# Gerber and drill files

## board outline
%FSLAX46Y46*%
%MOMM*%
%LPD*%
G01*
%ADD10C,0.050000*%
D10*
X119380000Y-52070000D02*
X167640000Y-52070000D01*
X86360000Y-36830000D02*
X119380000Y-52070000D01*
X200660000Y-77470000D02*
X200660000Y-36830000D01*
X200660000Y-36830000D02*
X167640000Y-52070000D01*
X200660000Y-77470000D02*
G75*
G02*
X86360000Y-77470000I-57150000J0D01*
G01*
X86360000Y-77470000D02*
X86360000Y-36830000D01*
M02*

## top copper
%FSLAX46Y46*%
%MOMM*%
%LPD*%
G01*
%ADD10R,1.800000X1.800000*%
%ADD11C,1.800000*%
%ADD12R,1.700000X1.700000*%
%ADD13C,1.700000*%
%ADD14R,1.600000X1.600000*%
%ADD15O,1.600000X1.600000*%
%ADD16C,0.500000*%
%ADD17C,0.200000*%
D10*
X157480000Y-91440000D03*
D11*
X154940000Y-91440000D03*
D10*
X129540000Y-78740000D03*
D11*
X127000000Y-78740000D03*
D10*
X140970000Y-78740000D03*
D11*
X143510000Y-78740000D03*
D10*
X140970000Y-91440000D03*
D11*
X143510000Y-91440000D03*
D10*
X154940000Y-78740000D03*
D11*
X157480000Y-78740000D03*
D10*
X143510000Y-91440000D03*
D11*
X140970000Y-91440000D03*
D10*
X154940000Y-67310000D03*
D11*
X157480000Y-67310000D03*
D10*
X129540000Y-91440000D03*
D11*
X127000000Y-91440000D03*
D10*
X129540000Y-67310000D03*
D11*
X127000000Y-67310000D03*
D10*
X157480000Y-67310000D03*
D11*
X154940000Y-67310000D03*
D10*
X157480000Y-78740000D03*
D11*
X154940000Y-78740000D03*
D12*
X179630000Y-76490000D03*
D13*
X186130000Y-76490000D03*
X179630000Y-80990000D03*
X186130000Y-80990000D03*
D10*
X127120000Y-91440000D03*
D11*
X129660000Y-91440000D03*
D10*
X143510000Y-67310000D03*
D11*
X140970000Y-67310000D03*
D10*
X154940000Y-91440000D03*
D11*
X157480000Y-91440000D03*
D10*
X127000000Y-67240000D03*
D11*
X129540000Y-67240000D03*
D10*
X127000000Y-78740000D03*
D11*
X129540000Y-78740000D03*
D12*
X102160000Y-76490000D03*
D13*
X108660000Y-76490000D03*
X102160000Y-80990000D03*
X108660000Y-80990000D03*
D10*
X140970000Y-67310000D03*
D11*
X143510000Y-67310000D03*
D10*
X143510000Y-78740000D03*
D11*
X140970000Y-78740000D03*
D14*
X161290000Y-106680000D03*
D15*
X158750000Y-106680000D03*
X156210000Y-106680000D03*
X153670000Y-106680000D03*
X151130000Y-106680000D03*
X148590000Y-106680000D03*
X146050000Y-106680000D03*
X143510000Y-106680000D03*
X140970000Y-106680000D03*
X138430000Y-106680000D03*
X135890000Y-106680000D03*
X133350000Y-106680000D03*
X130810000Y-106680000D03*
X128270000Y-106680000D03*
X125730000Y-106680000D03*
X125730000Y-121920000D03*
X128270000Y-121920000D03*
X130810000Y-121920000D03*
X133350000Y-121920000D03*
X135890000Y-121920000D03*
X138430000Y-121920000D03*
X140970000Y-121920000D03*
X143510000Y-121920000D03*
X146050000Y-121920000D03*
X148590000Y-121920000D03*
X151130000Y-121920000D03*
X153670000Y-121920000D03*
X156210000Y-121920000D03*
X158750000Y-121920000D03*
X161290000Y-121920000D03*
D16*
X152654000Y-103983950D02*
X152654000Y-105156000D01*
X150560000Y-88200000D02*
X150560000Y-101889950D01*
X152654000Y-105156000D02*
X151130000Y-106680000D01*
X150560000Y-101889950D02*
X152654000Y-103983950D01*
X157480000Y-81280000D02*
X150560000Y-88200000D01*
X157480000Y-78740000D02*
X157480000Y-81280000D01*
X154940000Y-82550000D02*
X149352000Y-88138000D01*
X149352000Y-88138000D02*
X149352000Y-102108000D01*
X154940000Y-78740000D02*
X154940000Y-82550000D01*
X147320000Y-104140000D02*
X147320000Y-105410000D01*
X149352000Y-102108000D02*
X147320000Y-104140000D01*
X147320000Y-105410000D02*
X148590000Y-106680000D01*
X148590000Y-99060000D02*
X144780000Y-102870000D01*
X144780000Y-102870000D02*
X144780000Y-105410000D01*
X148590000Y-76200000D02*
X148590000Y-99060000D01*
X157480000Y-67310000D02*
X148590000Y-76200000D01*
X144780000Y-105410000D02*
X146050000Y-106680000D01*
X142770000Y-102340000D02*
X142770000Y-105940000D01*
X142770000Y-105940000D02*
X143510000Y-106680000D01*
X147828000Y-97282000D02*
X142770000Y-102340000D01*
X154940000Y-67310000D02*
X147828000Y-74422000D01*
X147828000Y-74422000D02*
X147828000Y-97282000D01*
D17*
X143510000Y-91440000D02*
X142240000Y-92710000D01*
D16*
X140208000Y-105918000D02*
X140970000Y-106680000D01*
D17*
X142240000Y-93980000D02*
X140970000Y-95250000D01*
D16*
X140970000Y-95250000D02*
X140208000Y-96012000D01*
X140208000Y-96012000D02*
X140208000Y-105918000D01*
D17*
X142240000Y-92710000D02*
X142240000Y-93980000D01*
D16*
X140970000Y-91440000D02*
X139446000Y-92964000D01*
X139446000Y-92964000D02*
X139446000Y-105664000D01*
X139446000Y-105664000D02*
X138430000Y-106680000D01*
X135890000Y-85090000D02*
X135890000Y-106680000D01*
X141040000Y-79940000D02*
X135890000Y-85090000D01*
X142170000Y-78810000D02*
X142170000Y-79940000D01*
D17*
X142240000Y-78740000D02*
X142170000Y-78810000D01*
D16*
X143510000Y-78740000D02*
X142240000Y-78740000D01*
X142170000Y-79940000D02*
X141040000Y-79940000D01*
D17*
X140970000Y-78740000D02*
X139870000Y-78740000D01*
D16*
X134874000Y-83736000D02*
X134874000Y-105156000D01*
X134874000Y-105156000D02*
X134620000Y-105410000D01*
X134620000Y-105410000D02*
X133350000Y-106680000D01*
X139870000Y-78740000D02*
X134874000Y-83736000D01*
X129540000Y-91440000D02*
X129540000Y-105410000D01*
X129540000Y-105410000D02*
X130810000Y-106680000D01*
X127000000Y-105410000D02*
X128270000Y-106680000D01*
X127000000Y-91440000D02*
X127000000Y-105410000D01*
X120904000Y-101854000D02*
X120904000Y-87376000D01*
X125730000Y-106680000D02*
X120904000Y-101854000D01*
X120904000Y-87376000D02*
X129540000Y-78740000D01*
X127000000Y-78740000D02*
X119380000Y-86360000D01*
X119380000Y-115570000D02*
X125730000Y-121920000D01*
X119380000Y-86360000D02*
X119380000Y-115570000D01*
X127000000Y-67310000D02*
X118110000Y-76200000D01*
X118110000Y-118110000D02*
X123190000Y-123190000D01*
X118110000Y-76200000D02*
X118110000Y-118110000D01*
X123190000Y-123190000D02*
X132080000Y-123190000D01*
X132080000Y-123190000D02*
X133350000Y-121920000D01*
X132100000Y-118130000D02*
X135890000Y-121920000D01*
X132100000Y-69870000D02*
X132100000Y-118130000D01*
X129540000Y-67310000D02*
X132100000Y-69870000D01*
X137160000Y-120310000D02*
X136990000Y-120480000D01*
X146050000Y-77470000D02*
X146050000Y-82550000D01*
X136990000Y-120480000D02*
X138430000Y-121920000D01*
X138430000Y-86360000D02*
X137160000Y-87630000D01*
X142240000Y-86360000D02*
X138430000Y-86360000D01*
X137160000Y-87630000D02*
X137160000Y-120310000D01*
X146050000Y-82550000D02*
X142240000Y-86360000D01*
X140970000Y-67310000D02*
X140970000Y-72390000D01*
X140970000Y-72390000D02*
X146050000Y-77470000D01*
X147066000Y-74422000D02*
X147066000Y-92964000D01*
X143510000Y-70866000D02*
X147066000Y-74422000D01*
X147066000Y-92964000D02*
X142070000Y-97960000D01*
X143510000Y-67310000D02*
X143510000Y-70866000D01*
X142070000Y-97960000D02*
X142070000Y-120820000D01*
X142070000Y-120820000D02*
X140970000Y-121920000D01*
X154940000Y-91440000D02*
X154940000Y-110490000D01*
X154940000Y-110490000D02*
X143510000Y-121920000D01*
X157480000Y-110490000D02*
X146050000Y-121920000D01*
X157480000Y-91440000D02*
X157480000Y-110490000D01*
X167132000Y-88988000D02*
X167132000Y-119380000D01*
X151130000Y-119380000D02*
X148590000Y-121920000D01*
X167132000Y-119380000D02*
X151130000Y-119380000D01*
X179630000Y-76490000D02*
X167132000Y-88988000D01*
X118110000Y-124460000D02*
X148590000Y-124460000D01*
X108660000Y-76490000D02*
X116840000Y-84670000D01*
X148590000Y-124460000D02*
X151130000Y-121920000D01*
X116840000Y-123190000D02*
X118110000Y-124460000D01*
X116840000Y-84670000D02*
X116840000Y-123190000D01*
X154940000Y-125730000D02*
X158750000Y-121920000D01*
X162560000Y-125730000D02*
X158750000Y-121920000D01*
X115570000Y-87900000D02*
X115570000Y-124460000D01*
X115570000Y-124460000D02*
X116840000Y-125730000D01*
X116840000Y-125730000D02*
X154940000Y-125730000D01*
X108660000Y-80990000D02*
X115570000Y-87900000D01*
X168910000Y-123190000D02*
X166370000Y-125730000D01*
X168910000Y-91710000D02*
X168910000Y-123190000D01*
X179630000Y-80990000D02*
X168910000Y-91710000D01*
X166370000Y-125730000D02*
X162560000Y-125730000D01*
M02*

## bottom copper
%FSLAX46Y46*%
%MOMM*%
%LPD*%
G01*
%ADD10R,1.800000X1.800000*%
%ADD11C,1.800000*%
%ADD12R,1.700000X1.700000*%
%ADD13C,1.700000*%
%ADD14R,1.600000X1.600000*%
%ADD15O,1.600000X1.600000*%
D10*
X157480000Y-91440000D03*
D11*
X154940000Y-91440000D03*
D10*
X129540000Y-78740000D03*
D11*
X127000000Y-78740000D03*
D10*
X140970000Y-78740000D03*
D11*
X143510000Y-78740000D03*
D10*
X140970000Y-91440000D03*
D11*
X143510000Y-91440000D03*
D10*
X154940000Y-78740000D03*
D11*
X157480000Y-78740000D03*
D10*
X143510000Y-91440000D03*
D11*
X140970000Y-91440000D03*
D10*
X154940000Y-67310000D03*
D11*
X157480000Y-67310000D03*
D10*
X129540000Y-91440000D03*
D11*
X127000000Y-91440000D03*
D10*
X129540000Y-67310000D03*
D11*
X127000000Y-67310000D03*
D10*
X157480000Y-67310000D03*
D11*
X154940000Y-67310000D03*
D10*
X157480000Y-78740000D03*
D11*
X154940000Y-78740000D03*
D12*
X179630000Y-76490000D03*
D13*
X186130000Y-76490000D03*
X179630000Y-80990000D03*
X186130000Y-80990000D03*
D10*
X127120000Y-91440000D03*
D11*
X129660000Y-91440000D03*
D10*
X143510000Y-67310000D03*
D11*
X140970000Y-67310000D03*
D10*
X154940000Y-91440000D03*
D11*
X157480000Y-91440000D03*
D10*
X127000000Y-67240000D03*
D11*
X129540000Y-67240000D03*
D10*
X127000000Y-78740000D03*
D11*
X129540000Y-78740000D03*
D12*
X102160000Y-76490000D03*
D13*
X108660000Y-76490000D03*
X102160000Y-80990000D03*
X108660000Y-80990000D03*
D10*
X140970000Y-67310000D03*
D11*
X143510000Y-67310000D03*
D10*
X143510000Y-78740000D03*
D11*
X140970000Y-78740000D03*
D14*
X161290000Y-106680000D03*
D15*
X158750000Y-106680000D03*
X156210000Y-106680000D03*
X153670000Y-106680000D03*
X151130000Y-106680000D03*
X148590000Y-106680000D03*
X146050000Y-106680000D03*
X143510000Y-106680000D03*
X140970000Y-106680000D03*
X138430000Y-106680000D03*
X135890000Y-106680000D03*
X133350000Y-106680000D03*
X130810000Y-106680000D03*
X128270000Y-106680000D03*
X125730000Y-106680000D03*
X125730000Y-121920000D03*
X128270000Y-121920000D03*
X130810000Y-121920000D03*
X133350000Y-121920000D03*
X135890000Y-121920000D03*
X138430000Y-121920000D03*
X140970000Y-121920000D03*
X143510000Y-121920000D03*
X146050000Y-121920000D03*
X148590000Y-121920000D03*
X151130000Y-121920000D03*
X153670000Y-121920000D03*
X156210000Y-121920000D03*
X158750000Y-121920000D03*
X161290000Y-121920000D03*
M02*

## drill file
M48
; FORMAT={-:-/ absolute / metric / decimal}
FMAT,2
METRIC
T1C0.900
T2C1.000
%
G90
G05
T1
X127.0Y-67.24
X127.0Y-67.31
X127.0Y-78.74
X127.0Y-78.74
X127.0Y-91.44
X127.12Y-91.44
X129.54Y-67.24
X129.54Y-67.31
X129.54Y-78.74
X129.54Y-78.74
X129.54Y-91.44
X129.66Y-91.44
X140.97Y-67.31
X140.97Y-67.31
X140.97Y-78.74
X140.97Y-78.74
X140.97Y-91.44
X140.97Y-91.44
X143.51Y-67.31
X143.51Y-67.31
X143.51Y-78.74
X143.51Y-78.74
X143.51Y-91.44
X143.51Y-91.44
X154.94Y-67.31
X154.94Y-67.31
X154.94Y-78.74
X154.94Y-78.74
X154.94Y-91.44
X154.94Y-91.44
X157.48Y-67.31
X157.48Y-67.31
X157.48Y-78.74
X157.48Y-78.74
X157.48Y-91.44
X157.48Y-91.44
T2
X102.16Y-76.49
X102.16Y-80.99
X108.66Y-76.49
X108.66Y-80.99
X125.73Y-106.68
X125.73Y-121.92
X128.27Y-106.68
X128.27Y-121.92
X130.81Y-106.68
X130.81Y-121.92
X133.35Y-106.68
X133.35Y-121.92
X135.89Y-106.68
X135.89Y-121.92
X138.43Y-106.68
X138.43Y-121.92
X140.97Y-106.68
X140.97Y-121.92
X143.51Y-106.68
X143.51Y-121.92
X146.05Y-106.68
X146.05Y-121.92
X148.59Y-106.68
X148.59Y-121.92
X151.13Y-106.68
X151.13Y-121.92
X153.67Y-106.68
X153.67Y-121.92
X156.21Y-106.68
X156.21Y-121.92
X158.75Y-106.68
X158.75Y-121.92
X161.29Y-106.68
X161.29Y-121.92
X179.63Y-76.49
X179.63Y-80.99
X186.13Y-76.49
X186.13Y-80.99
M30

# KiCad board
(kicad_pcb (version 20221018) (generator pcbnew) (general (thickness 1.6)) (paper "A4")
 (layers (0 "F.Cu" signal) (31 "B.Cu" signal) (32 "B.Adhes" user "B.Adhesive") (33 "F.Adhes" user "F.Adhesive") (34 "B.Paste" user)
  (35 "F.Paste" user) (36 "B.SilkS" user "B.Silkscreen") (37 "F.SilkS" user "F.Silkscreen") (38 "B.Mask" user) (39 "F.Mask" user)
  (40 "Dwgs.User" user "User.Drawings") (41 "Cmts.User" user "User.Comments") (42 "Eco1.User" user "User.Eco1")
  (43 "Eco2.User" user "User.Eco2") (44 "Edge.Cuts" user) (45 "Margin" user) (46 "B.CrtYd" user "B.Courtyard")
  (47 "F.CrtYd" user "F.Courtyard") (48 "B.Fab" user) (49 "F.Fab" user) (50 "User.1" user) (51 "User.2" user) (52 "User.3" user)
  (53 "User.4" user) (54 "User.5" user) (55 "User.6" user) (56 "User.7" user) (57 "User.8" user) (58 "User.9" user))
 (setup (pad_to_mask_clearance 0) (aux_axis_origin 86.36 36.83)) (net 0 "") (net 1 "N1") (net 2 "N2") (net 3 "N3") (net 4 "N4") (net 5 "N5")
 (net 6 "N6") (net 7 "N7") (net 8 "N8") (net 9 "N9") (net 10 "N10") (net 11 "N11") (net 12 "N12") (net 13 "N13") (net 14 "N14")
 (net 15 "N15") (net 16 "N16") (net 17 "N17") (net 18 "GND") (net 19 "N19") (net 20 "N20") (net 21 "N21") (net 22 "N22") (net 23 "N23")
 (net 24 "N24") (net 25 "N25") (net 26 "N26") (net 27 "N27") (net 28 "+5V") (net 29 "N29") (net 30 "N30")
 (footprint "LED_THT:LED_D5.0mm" (layer "F.Cu") (at 157.48 91.44 180)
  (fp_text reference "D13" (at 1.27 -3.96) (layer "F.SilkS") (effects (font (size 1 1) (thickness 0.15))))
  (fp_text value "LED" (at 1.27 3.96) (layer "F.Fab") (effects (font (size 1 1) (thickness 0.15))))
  (pad "1" thru_hole rect (at 0 0 180) (size 1.8 1.8) (drill 0.9) (layers "*.Cu" "*.Mask") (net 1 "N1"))
  (pad "2" thru_hole circle (at 2.54 0 180) (size 1.8 1.8) (drill 0.9) (layers "*.Cu" "*.Mask") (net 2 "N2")))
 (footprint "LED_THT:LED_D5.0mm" (layer "F.Cu") (at 129.54 78.74 180)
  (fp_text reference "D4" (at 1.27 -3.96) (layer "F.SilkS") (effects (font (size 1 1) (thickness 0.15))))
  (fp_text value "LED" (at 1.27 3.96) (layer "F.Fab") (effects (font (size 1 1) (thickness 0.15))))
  (pad "1" thru_hole rect (at 0 0 180) (size 1.8 1.8) (drill 0.9) (layers "*.Cu" "*.Mask") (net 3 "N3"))
  (pad "2" thru_hole circle (at 2.54 0 180) (size 1.8 1.8) (drill 0.9) (layers "*.Cu" "*.Mask") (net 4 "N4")))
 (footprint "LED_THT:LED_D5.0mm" (layer "F.Cu") (at 140.97 78.74)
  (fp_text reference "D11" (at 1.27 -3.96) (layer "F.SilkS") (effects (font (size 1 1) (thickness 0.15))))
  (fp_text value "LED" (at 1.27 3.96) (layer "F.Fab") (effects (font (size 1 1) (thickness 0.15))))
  (pad "1" thru_hole rect (at 0 0) (size 1.8 1.8) (drill 0.9) (layers "*.Cu" "*.Mask") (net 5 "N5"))
  (pad "2" thru_hole circle (at 2.54 0) (size 1.8 1.8) (drill 0.9) (layers "*.Cu" "*.Mask") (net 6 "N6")))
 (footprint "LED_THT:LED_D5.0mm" (layer "F.Cu") (at 140.97 91.44)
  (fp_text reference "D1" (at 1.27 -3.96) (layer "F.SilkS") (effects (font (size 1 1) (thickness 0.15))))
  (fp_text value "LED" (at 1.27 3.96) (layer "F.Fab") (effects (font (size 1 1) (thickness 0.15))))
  (pad "1" thru_hole rect (at 0 0) (size 1.8 1.8) (drill 0.9) (layers "*.Cu" "*.Mask") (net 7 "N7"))
  (pad "2" thru_hole circle (at 2.54 0) (size 1.8 1.8) (drill 0.9) (layers "*.Cu" "*.Mask") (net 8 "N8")))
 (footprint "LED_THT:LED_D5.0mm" (layer "F.Cu") (at 154.94 78.74)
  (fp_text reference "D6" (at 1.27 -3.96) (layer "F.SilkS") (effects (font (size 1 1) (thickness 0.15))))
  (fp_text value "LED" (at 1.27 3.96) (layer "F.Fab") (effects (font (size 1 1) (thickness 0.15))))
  (pad "1" thru_hole rect (at 0 0) (size 1.8 1.8) (drill 0.9) (layers "*.Cu" "*.Mask") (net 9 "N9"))
  (pad "2" thru_hole circle (at 2.54 0) (size 1.8 1.8) (drill 0.9) (layers "*.Cu" "*.Mask") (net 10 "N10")))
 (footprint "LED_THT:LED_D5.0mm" (layer "F.Cu") (at 143.51 91.44 180)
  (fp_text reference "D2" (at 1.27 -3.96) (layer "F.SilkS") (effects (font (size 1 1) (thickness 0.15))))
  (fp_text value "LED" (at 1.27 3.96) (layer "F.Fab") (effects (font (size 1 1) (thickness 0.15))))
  (pad "1" thru_hole rect (at 0 0 180) (size 1.8 1.8) (drill 0.9) (layers "*.Cu" "*.Mask") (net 8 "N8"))
  (pad "2" thru_hole circle (at 2.54 0 180) (size 1.8 1.8) (drill 0.9) (layers "*.Cu" "*.Mask") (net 7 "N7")))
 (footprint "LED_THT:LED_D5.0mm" (layer "F.Cu") (at 154.94 67.31)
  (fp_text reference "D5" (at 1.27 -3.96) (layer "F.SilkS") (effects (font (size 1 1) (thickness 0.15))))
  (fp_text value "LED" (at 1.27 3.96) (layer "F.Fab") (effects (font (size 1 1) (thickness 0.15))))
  (pad "1" thru_hole rect (at 0 0) (size 1.8 1.8) (drill 0.9) (layers "*.Cu" "*.Mask") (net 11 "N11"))
  (pad "2" thru_hole circle (at 2.54 0) (size 1.8 1.8) (drill 0.9) (layers "*.Cu" "*.Mask") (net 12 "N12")))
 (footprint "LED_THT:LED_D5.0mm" (layer "F.Cu") (at 129.54 91.44 180)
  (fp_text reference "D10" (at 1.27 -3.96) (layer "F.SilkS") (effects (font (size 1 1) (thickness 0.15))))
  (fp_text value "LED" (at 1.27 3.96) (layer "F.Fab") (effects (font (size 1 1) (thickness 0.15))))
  (pad "1" thru_hole rect (at 0 0 180) (size 1.8 1.8) (drill 0.9) (layers "*.Cu" "*.Mask") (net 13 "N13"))
  (pad "2" thru_hole circle (at 2.54 0 180) (size 1.8 1.8) (drill 0.9) (layers "*.Cu" "*.Mask") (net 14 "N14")))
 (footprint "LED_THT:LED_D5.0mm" (layer "F.Cu") (at 129.54 67.31 180)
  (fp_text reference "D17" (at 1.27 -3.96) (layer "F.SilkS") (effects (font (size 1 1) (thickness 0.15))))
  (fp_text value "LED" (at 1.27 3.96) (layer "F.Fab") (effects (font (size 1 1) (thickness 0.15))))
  (pad "1" thru_hole rect (at 0 0 180) (size 1.8 1.8) (drill 0.9) (layers "*.Cu" "*.Mask") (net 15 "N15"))
  (pad "2" thru_hole circle (at 2.54 0 180) (size 1.8 1.8) (drill 0.9) (layers "*.Cu" "*.Mask") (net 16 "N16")))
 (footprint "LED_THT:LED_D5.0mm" (layer "F.Cu") (at 157.48 67.31 180)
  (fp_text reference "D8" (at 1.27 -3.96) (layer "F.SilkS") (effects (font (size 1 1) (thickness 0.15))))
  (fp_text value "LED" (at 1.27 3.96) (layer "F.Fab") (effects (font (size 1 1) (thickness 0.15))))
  (pad "1" thru_hole rect (at 0 0 180) (size 1.8 1.8) (drill 0.9) (layers "*.Cu" "*.Mask") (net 12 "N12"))
  (pad "2" thru_hole circle (at 2.54 0 180) (size 1.8 1.8) (drill 0.9) (layers "*.Cu" "*.Mask") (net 11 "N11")))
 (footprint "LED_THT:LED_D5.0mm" (layer "F.Cu") (at 157.48 78.74 180)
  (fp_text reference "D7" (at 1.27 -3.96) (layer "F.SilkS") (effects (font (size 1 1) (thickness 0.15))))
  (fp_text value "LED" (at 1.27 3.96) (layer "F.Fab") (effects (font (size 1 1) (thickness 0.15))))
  (pad "1" thru_hole rect (at 0 0 180) (size 1.8 1.8) (drill 0.9) (layers "*.Cu" "*.Mask") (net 10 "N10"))
  (pad "2" thru_hole circle (at 2.54 0 180) (size 1.8 1.8) (drill 0.9) (layers "*.Cu" "*.Mask") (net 9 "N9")))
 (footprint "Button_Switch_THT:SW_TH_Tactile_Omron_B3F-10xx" (layer "F.Cu") (at 179.63 76.49)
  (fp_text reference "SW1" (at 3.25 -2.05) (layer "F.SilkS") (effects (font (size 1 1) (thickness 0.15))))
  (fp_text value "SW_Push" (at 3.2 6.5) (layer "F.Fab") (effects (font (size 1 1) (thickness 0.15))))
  (pad "1" thru_hole rect (at 0 0) (size 1.7 1.7) (drill 1) (layers "*.Cu" "*.Mask") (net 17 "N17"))
  (pad "1" thru_hole circle (at 6.5 0) (size 1.7 1.7) (drill 1) (layers "*.Cu" "*.Mask") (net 17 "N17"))
  (pad "2" thru_hole circle (at 0 4.5) (size 1.7 1.7) (drill 1) (layers "*.Cu" "*.Mask") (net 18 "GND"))
  (pad "2" thru_hole circle (at 6.5 4.5) (size 1.7 1.7) (drill 1) (layers "*.Cu" "*.Mask") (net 18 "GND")))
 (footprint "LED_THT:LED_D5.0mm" (layer "F.Cu") (at 127.12 91.44)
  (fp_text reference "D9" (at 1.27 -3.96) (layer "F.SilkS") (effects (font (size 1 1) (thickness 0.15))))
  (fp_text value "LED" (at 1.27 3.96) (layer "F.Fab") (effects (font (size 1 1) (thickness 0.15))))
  (pad "1" thru_hole rect (at 0 0) (size 1.8 1.8) (drill 0.9) (layers "*.Cu" "*.Mask") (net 14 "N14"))
  (pad "2" thru_hole circle (at 2.54 0) (size 1.8 1.8) (drill 0.9) (layers "*.Cu" "*.Mask") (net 13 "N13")))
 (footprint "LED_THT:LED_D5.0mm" (layer "F.Cu") (at 143.51 67.31 180)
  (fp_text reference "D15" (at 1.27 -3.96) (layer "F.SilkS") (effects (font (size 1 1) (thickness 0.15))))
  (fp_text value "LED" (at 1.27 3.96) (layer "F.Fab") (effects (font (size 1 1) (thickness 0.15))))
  (pad "1" thru_hole rect (at 0 0 180) (size 1.8 1.8) (drill 0.9) (layers "*.Cu" "*.Mask") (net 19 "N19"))
  (pad "2" thru_hole circle (at 2.54 0 180) (size 1.8 1.8) (drill 0.9) (layers "*.Cu" "*.Mask") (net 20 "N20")))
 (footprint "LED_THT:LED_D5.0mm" (layer "F.Cu") (at 154.94 91.44)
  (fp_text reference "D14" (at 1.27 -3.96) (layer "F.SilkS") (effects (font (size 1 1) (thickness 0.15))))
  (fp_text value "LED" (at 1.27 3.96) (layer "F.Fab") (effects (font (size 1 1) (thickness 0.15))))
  (pad "1" thru_hole rect (at 0 0) (size 1.8 1.8) (drill 0.9) (layers "*.Cu" "*.Mask") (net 2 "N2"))
  (pad "2" thru_hole circle (at 2.54 0) (size 1.8 1.8) (drill 0.9) (layers "*.Cu" "*.Mask") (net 1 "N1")))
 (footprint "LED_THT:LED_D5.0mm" (layer "F.Cu") (at 127 67.24)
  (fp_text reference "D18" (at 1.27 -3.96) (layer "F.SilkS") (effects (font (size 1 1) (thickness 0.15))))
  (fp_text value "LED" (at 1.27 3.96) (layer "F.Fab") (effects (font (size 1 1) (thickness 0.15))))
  (pad "1" thru_hole rect (at 0 0) (size 1.8 1.8) (drill 0.9) (layers "*.Cu" "*.Mask") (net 16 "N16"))
  (pad "2" thru_hole circle (at 2.54 0) (size 1.8 1.8) (drill 0.9) (layers "*.Cu" "*.Mask") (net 15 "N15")))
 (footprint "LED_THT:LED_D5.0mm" (layer "F.Cu") (at 127 78.74)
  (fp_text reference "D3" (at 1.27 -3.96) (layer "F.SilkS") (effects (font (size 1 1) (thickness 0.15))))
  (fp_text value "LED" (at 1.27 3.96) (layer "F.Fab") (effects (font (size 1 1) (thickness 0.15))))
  (pad "1" thru_hole rect (at 0 0) (size 1.8 1.8) (drill 0.9) (layers "*.Cu" "*.Mask") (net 4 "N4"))
  (pad "2" thru_hole circle (at 2.54 0) (size 1.8 1.8) (drill 0.9) (layers "*.Cu" "*.Mask") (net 3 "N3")))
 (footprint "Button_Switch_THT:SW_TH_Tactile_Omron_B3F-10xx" (layer "F.Cu") (at 102.16 76.49)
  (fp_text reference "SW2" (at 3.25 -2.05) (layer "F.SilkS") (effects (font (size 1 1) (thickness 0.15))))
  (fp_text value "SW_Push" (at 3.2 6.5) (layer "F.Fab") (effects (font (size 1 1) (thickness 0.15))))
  (pad "1" thru_hole rect (at 0 0) (size 1.7 1.7) (drill 1) (layers "*.Cu" "*.Mask") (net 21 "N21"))
  (pad "1" thru_hole circle (at 6.5 0) (size 1.7 1.7) (drill 1) (layers "*.Cu" "*.Mask") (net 21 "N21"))
  (pad "2" thru_hole circle (at 0 4.5) (size 1.7 1.7) (drill 1) (layers "*.Cu" "*.Mask") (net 18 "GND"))
  (pad "2" thru_hole circle (at 6.5 4.5) (size 1.7 1.7) (drill 1) (layers "*.Cu" "*.Mask") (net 18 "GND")))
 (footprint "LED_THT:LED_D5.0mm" (layer "F.Cu") (at 140.97 67.31)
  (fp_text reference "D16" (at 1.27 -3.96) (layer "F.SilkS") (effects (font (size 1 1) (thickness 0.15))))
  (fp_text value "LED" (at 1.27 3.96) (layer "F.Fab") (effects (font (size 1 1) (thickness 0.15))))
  (pad "1" thru_hole rect (at 0 0) (size 1.8 1.8) (drill 0.9) (layers "*.Cu" "*.Mask") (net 20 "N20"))
  (pad "2" thru_hole circle (at 2.54 0) (size 1.8 1.8) (drill 0.9) (layers "*.Cu" "*.Mask") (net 19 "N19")))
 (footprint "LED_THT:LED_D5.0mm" (layer "F.Cu") (at 143.51 78.74 180)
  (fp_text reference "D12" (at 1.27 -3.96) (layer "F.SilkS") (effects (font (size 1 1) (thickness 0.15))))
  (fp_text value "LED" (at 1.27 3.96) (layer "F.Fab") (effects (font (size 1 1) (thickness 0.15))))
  (pad "1" thru_hole rect (at 0 0 180) (size 1.8 1.8) (drill 0.9) (layers "*.Cu" "*.Mask") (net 6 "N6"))
  (pad "2" thru_hole circle (at 2.54 0 180) (size 1.8 1.8) (drill 0.9) (layers "*.Cu" "*.Mask") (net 5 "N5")))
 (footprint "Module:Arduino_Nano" (layer "F.Cu") (at 161.29 106.68 -90)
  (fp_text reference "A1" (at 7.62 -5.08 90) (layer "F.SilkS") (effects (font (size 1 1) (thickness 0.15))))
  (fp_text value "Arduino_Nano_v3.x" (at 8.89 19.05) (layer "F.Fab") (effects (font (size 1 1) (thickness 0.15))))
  (pad "1" thru_hole rect (at 0 0 270) (size 1.6 1.6) (drill 1) (layers "*.Cu" "*.Mask") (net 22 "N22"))
  (pad "2" thru_hole oval (at 0 2.54 270) (size 1.6 1.6) (drill 1) (layers "*.Cu" "*.Mask") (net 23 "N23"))
  (pad "3" thru_hole oval (at 0 5.08 270) (size 1.6 1.6) (drill 1) (layers "*.Cu" "*.Mask") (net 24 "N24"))
  (pad "4" thru_hole oval (at 0 7.62 270) (size 1.6 1.6) (drill 1) (layers "*.Cu" "*.Mask") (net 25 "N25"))
  (pad "5" thru_hole oval (at 0 10.16 270) (size 1.6 1.6) (drill 1) (layers "*.Cu" "*.Mask") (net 10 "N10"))
  (pad "6" thru_hole oval (at 0 12.7 270) (size 1.6 1.6) (drill 1) (layers "*.Cu" "*.Mask") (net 9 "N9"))
  (pad "7" thru_hole oval (at 0 15.24 270) (size 1.6 1.6) (drill 1) (layers "*.Cu" "*.Mask") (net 12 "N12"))
  (pad "8" thru_hole oval (at 0 17.78 270) (size 1.6 1.6) (drill 1) (layers "*.Cu" "*.Mask") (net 11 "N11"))
  (pad "9" thru_hole oval (at 0 20.32 270) (size 1.6 1.6) (drill 1) (layers "*.Cu" "*.Mask") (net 8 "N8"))
  (pad "10" thru_hole oval (at 0 22.86 270) (size 1.6 1.6) (drill 1) (layers "*.Cu" "*.Mask") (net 7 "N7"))
  (pad "11" thru_hole oval (at 0 25.4 270) (size 1.6 1.6) (drill 1) (layers "*.Cu" "*.Mask") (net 6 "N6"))
  (pad "12" thru_hole oval (at 0 27.94 270) (size 1.6 1.6) (drill 1) (layers "*.Cu" "*.Mask") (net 5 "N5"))
  (pad "13" thru_hole oval (at 0 30.48 270) (size 1.6 1.6) (drill 1) (layers "*.Cu" "*.Mask") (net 13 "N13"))
  (pad "14" thru_hole oval (at 0 33.02 270) (size 1.6 1.6) (drill 1) (layers "*.Cu" "*.Mask") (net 14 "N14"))
  (pad "15" thru_hole oval (at 0 35.56 270) (size 1.6 1.6) (drill 1) (layers "*.Cu" "*.Mask") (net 3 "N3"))
  (pad "16" thru_hole oval (at 15.24 35.56 270) (size 1.6 1.6) (drill 1) (layers "*.Cu" "*.Mask") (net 4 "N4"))
  (pad "17" thru_hole oval (at 15.24 33.02 270) (size 1.6 1.6) (drill 1) (layers "*.Cu" "*.Mask") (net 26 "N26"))
  (pad "18" thru_hole oval (at 15.24 30.48 270) (size 1.6 1.6) (drill 1) (layers "*.Cu" "*.Mask") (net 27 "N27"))
  (pad "19" thru_hole oval (at 15.24 27.94 270) (size 1.6 1.6) (drill 1) (layers "*.Cu" "*.Mask") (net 16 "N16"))
  (pad "20" thru_hole oval (at 15.24 25.4 270) (size 1.6 1.6) (drill 1) (layers "*.Cu" "*.Mask") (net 15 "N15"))
  (pad "21" thru_hole oval (at 15.24 22.86 270) (size 1.6 1.6) (drill 1) (layers "*.Cu" "*.Mask") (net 20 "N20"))
  (pad "22" thru_hole oval (at 15.24 20.32 270) (size 1.6 1.6) (drill 1) (layers "*.Cu" "*.Mask") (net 19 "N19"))
  (pad "23" thru_hole oval (at 15.24 17.78 270) (size 1.6 1.6) (drill 1) (layers "*.Cu" "*.Mask") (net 2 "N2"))
  (pad "24" thru_hole oval (at 15.24 15.24 270) (size 1.6 1.6) (drill 1) (layers "*.Cu" "*.Mask") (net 1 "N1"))
  (pad "25" thru_hole oval (at 15.24 12.7 270) (size 1.6 1.6) (drill 1) (layers "*.Cu" "*.Mask") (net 17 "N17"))
  (pad "26" thru_hole oval (at 15.24 10.16 270) (size 1.6 1.6) (drill 1) (layers "*.Cu" "*.Mask") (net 21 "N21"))
  (pad "27" thru_hole oval (at 15.24 7.62 270) (size 1.6 1.6) (drill 1) (layers "*.Cu" "*.Mask") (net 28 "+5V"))
  (pad "28" thru_hole oval (at 15.24 5.08 270) (size 1.6 1.6) (drill 1) (layers "*.Cu" "*.Mask") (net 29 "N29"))
  (pad "29" thru_hole oval (at 15.24 2.54 270) (size 1.6 1.6) (drill 1) (layers "*.Cu" "*.Mask") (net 18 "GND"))
  (pad "30" thru_hole oval (at 15.24 0 270) (size 1.6 1.6) (drill 1) (layers "*.Cu" "*.Mask") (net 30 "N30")))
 (gr_line (start 119.38 52.07) (end 167.64 52.07) (stroke (width 0.05) (type default)) (layer "Edge.Cuts"))
 (gr_line (start 86.36 36.83) (end 119.38 52.07) (stroke (width 0.05) (type default)) (layer "Edge.Cuts"))
 (gr_line (start 200.66 77.47) (end 200.66 36.83) (stroke (width 0.05) (type default)) (layer "Edge.Cuts"))
 (gr_line (start 200.66 36.83) (end 167.64 52.07) (stroke (width 0.05) (type default)) (layer "Edge.Cuts"))
 (gr_arc (start 200.66 77.47) (mid 143.51 134.62) (end 86.36 77.47) (stroke (width 0.05) (type default)) (layer "Edge.Cuts"))
 (gr_line (start 86.36 77.47) (end 86.36 36.83) (stroke (width 0.05) (type default)) (layer "Edge.Cuts"))
 (segment (start 152.654 103.98395) (end 152.654 105.156) (width 0.5) (layer "F.Cu") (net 10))
 (segment (start 150.56 88.2) (end 150.56 101.88995) (width 0.5) (layer "F.Cu") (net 10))
 (segment (start 152.654 105.156) (end 151.13 106.68) (width 0.5) (layer "F.Cu") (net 10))
 (segment (start 150.56 101.88995) (end 152.654 103.98395) (width 0.5) (layer "F.Cu") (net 10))
 (segment (start 157.48 81.28) (end 150.56 88.2) (width 0.5) (layer "F.Cu") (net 10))
 (segment (start 157.48 78.74) (end 157.48 81.28) (width 0.5) (layer "F.Cu") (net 10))
 (segment (start 154.94 82.55) (end 149.352 88.138) (width 0.5) (layer "F.Cu") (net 9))
 (segment (start 149.352 88.138) (end 149.352 102.108) (width 0.5) (layer "F.Cu") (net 9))
 (segment (start 154.94 78.74) (end 154.94 82.55) (width 0.5) (layer "F.Cu") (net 9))
 (segment (start 147.32 104.14) (end 147.32 105.41) (width 0.5) (layer "F.Cu") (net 9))
 (segment (start 149.352 102.108) (end 147.32 104.14) (width 0.5) (layer "F.Cu") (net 9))
 (segment (start 147.32 105.41) (end 148.59 106.68) (width 0.5) (layer "F.Cu") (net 9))
 (segment (start 148.59 99.06) (end 144.78 102.87) (width 0.5) (layer "F.Cu") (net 12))
 (segment (start 144.78 102.87) (end 144.78 105.41) (width 0.5) (layer "F.Cu") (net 12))
 (segment (start 148.59 76.2) (end 148.59 99.06) (width 0.5) (layer "F.Cu") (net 12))
 (segment (start 157.48 67.31) (end 148.59 76.2) (width 0.5) (layer "F.Cu") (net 12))
 (segment (start 144.78 105.41) (end 146.05 106.68) (width 0.5) (layer "F.Cu") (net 12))
 (segment (start 142.77 102.34) (end 142.77 105.94) (width 0.5) (layer "F.Cu") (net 11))
 (segment (start 142.77 105.94) (end 143.51 106.68) (width 0.5) (layer "F.Cu") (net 11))
 (segment (start 147.828 97.282) (end 142.77 102.34) (width 0.5) (layer "F.Cu") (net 11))
 (segment (start 154.94 67.31) (end 147.828 74.422) (width 0.5) (layer "F.Cu") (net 11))
 (segment (start 147.828 74.422) (end 147.828 97.282) (width 0.5) (layer "F.Cu") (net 11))
 (segment (start 143.51 91.44) (end 142.24 92.71) (width 0.2) (layer "F.Cu") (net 8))
 (segment (start 140.208 105.918) (end 140.97 106.68) (width 0.5) (layer "F.Cu") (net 8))
 (segment (start 142.24 93.98) (end 140.97 95.25) (width 0.2) (layer "F.Cu") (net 8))
 (segment (start 140.97 95.25) (end 140.208 96.012) (width 0.5) (layer "F.Cu") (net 8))
 (segment (start 140.208 96.012) (end 140.208 105.918) (width 0.5) (layer "F.Cu") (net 8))
 (segment (start 142.24 92.71) (end 142.24 93.98) (width 0.2) (layer "F.Cu") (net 8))
 (segment (start 140.97 91.44) (end 139.446 92.964) (width 0.5) (layer "F.Cu") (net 7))
 (segment (start 139.446 92.964) (end 139.446 105.664) (width 0.5) (layer "F.Cu") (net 7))
 (segment (start 139.446 105.664) (end 138.43 106.68) (width 0.5) (layer "F.Cu") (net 7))
 (segment (start 135.89 85.09) (end 135.89 106.68) (width 0.5) (layer "F.Cu") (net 6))
 (segment (start 141.04 79.94) (end 135.89 85.09) (width 0.5) (layer "F.Cu") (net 6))
 (segment (start 142.17 78.81) (end 142.17 79.94) (width 0.5) (layer "F.Cu") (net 6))
 (segment (start 142.24 78.74) (end 142.17 78.81) (width 0.2) (layer "F.Cu") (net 6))
 (segment (start 143.51 78.74) (end 142.24 78.74) (width 0.5) (layer "F.Cu") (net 6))
 (segment (start 142.17 79.94) (end 141.04 79.94) (width 0.5) (layer "F.Cu") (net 6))
 (segment (start 140.97 78.74) (end 139.87 78.74) (width 0.2) (layer "F.Cu") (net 5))
 (segment (start 134.874 83.736) (end 134.874 105.156) (width 0.5) (layer "F.Cu") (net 5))
 (segment (start 134.874 105.156) (end 134.62 105.41) (width 0.5) (layer "F.Cu") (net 5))
 (segment (start 134.62 105.41) (end 133.35 106.68) (width 0.5) (layer "F.Cu") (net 5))
 (segment (start 139.87 78.74) (end 134.874 83.736) (width 0.5) (layer "F.Cu") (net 5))
 (segment (start 129.54 91.44) (end 129.54 105.41) (width 0.5) (layer "F.Cu") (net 13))
 (segment (start 129.54 105.41) (end 130.81 106.68) (width 0.5) (layer "F.Cu") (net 13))
 (segment (start 127 105.41) (end 128.27 106.68) (width 0.5) (layer "F.Cu") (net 14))
 (segment (start 127 91.44) (end 127 105.41) (width 0.5) (layer "F.Cu") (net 14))
 (segment (start 120.904 101.854) (end 120.904 87.376) (width 0.5) (layer "F.Cu") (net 3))
 (segment (start 125.73 106.68) (end 120.904 101.854) (width 0.5) (layer "F.Cu") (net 3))
 (segment (start 120.904 87.376) (end 129.54 78.74) (width 0.5) (layer "F.Cu") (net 3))
 (segment (start 127 78.74) (end 119.38 86.36) (width 0.5) (layer "F.Cu") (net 4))
 (segment (start 119.38 115.57) (end 125.73 121.92) (width 0.5) (layer "F.Cu") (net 4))
 (segment (start 119.38 86.36) (end 119.38 115.57) (width 0.5) (layer "F.Cu") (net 4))
 (segment (start 127 67.31) (end 118.11 76.2) (width 0.5) (layer "F.Cu") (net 16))
 (segment (start 118.11 118.11) (end 123.19 123.19) (width 0.5) (layer "F.Cu") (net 16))
 (segment (start 118.11 76.2) (end 118.11 118.11) (width 0.5) (layer "F.Cu") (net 16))
 (segment (start 123.19 123.19) (end 132.08 123.19) (width 0.5) (layer "F.Cu") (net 16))
 (segment (start 132.08 123.19) (end 133.35 121.92) (width 0.5) (layer "F.Cu") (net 16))
 (segment (start 132.1 118.13) (end 135.89 121.92) (width 0.5) (layer "F.Cu") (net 15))
 (segment (start 132.1 69.87) (end 132.1 118.13) (width 0.5) (layer "F.Cu") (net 15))
 (segment (start 129.54 67.31) (end 132.1 69.87) (width 0.5) (layer "F.Cu") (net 15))
 (segment (start 137.16 120.31) (end 136.99 120.48) (width 0.5) (layer "F.Cu") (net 20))
 (segment (start 146.05 77.47) (end 146.05 82.55) (width 0.5) (layer "F.Cu") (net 20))
 (segment (start 136.99 120.48) (end 138.43 121.92) (width 0.5) (layer "F.Cu") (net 20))
 (segment (start 138.43 86.36) (end 137.16 87.63) (width 0.5) (layer "F.Cu") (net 20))
 (segment (start 142.24 86.36) (end 138.43 86.36) (width 0.5) (layer "F.Cu") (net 20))
 (segment (start 137.16 87.63) (end 137.16 120.31) (width 0.5) (layer "F.Cu") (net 20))
 (segment (start 146.05 82.55) (end 142.24 86.36) (width 0.5) (layer "F.Cu") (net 20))
 (segment (start 140.97 67.31) (end 140.97 72.39) (width 0.5) (layer "F.Cu") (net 20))
 (segment (start 140.97 72.39) (end 146.05 77.47) (width 0.5) (layer "F.Cu") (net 20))
 (segment (start 147.066 74.422) (end 147.066 92.964) (width 0.5) (layer "F.Cu") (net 19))
 (segment (start 143.51 70.866) (end 147.066 74.422) (width 0.5) (layer "F.Cu") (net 19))
 (segment (start 147.066 92.964) (end 142.07 97.96) (width 0.5) (layer "F.Cu") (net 19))
 (segment (start 143.51 67.31) (end 143.51 70.866) (width 0.5) (layer "F.Cu") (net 19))
 (segment (start 142.07 97.96) (end 142.07 120.82) (width 0.5) (layer "F.Cu") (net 19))
 (segment (start 142.07 120.82) (end 140.97 121.92) (width 0.5) (layer "F.Cu") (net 19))
 (segment (start 154.94 91.44) (end 154.94 110.49) (width 0.5) (layer "F.Cu") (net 2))
 (segment (start 154.94 110.49) (end 143.51 121.92) (width 0.5) (layer "F.Cu") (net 2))
 (segment (start 157.48 110.49) (end 146.05 121.92) (width 0.5) (layer "F.Cu") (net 1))
 (segment (start 157.48 91.44) (end 157.48 110.49) (width 0.5) (layer "F.Cu") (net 1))
 (segment (start 167.132 88.988) (end 167.132 119.38) (width 0.5) (layer "F.Cu") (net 17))
 (segment (start 151.13 119.38) (end 148.59 121.92) (width 0.5) (layer "F.Cu") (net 17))
 (segment (start 167.132 119.38) (end 151.13 119.38) (width 0.5) (layer "F.Cu") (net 17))
 (segment (start 179.63 76.49) (end 167.132 88.988) (width 0.5) (layer "F.Cu") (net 17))
 (segment (start 118.11 124.46) (end 148.59 124.46) (width 0.5) (layer "F.Cu") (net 21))
 (segment (start 108.66 76.49) (end 116.84 84.67) (width 0.5) (layer "F.Cu") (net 21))
 (segment (start 148.59 124.46) (end 151.13 121.92) (width 0.5) (layer "F.Cu") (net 21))
 (segment (start 116.84 123.19) (end 118.11 124.46) (width 0.5) (layer "F.Cu") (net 21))
 (segment (start 116.84 84.67) (end 116.84 123.19) (width 0.5) (layer "F.Cu") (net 21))
 (segment (start 154.94 125.73) (end 158.75 121.92) (width 0.5) (layer "F.Cu") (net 18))
 (segment (start 162.56 125.73) (end 158.75 121.92) (width 0.5) (layer "F.Cu") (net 18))
 (segment (start 115.57 87.9) (end 115.57 124.46) (width 0.5) (layer "F.Cu") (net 18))
 (segment (start 115.57 124.46) (end 116.84 125.73) (width 0.5) (layer "F.Cu") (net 18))
 (segment (start 116.84 125.73) (end 154.94 125.73) (width 0.5) (layer "F.Cu") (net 18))
 (segment (start 108.66 80.99) (end 115.57 87.9) (width 0.5) (layer "F.Cu") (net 18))
 (segment (start 168.91 123.19) (end 166.37 125.73) (width 0.5) (layer "F.Cu") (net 18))
 (segment (start 168.91 91.71) (end 168.91 123.19) (width 0.5) (layer "F.Cu") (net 18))
 (segment (start 179.63 80.99) (end 168.91 91.71) (width 0.5) (layer "F.Cu") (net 18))
 (segment (start 166.37 125.73) (end 162.56 125.73) (width 0.5) (layer "F.Cu") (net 18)))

